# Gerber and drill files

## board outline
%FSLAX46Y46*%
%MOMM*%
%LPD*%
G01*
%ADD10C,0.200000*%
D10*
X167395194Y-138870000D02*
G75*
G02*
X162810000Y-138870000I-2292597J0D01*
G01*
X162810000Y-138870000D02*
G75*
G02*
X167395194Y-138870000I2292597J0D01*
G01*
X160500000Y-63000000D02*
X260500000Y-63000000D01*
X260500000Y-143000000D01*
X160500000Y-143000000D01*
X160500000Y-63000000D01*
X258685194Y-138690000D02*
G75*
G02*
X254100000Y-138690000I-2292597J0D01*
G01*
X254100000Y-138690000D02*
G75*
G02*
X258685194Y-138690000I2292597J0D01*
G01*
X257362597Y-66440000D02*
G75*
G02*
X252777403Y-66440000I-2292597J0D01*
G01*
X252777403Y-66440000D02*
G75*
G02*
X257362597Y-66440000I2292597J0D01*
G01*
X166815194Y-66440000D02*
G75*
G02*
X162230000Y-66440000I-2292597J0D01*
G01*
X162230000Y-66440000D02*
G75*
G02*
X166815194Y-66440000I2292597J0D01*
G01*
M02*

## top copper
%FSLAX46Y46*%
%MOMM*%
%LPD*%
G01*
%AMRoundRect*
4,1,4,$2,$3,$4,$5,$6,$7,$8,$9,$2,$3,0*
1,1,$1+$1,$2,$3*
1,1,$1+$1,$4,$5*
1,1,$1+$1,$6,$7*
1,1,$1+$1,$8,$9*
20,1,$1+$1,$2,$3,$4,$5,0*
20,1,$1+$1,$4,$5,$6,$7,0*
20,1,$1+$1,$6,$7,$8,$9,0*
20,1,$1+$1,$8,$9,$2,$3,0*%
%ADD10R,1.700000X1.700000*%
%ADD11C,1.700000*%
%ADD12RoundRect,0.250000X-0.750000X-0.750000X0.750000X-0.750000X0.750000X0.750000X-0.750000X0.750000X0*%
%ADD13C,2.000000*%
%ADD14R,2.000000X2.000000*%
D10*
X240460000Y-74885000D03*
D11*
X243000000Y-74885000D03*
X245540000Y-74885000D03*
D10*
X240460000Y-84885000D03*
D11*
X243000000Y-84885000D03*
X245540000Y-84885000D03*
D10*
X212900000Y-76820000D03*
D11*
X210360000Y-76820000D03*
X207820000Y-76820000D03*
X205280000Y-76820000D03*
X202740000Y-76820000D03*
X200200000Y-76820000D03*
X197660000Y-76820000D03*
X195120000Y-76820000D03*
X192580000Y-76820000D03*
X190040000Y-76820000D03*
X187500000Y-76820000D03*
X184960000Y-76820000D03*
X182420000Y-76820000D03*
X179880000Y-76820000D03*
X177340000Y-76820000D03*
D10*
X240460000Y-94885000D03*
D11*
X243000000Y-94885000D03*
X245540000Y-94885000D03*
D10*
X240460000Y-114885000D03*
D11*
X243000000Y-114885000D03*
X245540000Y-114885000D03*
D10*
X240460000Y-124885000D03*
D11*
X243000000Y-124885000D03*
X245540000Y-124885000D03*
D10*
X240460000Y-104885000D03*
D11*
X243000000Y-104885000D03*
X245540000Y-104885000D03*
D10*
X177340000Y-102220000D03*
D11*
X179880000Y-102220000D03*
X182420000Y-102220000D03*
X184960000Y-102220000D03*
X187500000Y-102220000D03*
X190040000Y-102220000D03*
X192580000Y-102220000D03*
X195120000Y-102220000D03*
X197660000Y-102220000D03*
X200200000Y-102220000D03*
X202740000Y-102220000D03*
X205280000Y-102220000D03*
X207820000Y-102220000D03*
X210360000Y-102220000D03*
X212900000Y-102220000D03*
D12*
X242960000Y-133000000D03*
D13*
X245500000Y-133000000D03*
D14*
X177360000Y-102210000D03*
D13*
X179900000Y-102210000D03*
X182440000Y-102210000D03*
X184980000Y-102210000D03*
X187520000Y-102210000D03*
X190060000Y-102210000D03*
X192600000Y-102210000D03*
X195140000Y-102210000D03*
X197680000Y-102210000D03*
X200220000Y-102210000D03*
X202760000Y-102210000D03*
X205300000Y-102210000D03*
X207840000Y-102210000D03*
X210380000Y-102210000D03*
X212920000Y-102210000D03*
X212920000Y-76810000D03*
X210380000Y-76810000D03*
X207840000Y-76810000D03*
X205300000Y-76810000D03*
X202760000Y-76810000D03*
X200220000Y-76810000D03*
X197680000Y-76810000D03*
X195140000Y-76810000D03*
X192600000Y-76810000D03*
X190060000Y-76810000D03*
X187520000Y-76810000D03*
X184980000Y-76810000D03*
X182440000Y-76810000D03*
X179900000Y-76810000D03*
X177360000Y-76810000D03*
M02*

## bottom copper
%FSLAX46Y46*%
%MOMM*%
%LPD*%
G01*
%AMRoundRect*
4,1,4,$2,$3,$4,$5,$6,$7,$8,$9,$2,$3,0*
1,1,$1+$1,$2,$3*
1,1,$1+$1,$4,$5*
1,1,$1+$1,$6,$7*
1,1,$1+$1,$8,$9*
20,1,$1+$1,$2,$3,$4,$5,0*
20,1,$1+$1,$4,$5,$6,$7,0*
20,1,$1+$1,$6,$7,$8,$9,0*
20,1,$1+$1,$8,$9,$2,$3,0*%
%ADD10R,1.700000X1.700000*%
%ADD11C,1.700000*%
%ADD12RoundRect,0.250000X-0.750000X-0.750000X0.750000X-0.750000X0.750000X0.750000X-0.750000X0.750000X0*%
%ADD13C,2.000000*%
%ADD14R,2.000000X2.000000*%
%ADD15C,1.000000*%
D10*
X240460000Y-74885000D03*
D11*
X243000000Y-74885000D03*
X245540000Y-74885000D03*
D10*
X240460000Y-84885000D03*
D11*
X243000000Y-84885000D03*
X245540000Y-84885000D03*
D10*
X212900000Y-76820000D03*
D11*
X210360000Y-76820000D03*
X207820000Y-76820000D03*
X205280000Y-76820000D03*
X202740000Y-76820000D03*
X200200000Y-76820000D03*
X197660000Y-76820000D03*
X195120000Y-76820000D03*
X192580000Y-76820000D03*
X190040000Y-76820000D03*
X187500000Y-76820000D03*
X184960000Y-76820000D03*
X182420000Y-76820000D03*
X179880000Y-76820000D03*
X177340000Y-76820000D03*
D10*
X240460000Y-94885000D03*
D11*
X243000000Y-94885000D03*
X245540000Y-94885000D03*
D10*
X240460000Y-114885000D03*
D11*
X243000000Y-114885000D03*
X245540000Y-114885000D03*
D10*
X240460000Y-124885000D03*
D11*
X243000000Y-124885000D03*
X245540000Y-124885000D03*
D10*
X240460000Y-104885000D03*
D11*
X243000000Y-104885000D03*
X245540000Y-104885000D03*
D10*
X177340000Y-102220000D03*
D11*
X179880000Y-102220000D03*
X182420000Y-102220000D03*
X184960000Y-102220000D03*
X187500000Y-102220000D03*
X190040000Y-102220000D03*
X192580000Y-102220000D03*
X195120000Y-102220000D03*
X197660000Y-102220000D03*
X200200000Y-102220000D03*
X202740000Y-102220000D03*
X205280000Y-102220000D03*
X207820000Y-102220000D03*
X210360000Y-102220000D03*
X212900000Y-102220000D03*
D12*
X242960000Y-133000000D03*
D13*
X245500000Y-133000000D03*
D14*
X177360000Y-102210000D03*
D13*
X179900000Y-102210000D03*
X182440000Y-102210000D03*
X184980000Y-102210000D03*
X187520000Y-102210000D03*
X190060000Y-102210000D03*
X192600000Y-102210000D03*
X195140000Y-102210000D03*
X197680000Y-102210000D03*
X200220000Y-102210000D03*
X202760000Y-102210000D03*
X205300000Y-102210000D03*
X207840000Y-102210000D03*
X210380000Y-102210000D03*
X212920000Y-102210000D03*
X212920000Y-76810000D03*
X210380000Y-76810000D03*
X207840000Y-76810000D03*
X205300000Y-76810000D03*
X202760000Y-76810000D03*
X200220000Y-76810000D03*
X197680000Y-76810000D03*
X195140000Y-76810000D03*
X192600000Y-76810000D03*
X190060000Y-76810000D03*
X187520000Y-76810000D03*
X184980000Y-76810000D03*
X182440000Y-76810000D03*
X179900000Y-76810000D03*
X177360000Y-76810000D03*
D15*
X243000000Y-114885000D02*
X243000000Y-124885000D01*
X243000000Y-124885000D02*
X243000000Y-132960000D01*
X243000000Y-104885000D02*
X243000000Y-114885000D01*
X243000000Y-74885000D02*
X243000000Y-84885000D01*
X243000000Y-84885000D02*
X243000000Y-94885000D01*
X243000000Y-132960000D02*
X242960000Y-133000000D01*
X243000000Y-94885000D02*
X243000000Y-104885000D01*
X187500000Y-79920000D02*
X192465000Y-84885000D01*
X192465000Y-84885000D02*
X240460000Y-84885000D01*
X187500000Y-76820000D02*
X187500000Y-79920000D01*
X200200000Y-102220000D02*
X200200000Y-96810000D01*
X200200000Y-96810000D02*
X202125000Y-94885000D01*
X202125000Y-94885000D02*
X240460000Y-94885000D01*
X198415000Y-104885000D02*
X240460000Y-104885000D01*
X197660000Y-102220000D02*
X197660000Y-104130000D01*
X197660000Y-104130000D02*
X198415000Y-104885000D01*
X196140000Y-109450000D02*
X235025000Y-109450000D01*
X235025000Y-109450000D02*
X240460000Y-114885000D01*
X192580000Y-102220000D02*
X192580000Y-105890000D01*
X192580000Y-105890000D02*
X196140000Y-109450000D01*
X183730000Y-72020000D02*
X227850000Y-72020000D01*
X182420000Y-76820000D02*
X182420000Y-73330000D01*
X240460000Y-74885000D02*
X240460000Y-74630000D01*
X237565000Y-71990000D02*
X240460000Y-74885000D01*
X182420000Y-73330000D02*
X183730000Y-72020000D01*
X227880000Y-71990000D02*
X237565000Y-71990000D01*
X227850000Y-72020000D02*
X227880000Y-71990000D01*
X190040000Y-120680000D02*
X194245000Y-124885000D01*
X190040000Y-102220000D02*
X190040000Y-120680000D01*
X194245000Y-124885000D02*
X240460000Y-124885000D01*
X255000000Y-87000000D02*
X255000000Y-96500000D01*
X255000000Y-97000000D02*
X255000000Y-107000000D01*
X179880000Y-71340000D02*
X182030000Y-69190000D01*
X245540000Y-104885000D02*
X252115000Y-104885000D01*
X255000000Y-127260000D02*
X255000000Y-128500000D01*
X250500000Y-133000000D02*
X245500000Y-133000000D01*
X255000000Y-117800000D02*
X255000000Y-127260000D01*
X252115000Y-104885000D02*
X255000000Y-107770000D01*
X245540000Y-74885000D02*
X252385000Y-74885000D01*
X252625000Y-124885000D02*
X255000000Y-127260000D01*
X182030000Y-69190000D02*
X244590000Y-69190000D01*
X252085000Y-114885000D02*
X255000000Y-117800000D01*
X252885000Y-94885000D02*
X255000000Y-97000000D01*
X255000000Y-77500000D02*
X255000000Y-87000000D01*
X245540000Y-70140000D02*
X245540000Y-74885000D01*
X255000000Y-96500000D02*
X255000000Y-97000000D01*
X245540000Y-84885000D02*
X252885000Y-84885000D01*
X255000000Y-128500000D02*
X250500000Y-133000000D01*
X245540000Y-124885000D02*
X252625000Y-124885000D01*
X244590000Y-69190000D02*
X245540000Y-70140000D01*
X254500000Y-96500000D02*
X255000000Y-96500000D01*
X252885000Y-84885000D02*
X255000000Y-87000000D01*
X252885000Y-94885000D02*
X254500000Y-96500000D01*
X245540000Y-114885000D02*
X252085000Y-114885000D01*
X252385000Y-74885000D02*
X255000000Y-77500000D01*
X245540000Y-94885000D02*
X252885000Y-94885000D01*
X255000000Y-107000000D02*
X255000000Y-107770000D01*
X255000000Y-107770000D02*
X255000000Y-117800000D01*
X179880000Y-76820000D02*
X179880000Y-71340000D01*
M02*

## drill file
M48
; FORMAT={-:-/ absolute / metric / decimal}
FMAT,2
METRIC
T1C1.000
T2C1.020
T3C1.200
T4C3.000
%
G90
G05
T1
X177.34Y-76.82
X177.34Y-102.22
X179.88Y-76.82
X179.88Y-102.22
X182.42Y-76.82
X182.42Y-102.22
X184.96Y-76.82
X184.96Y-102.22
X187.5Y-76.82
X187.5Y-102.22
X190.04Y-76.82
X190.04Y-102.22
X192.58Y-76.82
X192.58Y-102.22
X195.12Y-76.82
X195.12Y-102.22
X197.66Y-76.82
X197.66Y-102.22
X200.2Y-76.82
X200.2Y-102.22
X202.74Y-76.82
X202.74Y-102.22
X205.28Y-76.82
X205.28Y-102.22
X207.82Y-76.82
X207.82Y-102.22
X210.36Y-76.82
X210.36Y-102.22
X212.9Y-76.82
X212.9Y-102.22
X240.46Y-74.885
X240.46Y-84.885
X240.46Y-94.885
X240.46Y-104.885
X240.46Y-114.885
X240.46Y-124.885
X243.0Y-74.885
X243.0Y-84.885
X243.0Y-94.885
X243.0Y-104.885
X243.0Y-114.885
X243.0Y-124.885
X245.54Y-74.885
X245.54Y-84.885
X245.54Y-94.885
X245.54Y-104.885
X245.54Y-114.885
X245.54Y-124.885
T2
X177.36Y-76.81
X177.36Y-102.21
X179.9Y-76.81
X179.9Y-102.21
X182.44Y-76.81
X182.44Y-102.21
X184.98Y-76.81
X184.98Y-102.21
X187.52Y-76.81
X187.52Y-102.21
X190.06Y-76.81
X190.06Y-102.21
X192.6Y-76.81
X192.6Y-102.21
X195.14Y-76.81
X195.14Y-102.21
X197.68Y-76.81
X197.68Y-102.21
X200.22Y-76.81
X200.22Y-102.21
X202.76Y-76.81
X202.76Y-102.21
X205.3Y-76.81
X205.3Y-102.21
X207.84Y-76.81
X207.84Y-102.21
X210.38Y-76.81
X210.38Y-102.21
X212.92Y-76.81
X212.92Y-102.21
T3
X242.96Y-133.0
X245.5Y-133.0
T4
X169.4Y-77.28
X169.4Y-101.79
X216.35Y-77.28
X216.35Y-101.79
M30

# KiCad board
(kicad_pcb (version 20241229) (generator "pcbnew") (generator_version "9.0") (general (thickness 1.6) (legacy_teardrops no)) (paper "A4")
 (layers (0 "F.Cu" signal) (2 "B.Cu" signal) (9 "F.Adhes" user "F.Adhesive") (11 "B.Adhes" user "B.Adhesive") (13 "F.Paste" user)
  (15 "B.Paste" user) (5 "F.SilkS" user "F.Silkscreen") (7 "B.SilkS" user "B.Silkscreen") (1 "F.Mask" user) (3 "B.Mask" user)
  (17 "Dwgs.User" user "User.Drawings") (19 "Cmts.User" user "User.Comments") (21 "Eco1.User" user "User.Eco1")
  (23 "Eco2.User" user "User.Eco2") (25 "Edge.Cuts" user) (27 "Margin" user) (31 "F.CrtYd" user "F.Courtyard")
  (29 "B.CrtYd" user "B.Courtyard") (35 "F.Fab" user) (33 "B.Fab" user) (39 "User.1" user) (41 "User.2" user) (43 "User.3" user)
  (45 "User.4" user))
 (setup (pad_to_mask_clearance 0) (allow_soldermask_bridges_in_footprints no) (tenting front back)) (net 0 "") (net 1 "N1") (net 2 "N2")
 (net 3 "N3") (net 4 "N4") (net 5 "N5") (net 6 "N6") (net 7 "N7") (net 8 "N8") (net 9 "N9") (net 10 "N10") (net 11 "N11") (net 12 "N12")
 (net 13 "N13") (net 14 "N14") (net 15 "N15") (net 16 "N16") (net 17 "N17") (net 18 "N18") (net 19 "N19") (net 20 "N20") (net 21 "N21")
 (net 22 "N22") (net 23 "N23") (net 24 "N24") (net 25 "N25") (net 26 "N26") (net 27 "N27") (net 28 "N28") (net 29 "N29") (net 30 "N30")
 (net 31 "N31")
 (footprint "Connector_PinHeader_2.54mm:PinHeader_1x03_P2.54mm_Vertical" (layer "F.Cu") (at 240.46 74.885 90)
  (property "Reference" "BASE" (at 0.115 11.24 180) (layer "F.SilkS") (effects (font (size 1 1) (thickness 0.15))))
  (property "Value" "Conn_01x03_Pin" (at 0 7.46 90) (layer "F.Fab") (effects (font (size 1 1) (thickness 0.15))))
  (pad "1" thru_hole rect (at 0 0 90) (size 1.7 1.7) (drill 1) (layers "*.Cu" "*.Mask") (remove_unused_layers no) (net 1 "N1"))
  (pad "2" thru_hole circle (at 0 2.54 90) (size 1.7 1.7) (drill 1) (layers "*.Cu" "*.Mask") (remove_unused_layers no) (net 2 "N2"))
  (pad "3" thru_hole circle (at 0 5.08 90) (size 1.7 1.7) (drill 1) (layers "*.Cu" "*.Mask") (remove_unused_layers no) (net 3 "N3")))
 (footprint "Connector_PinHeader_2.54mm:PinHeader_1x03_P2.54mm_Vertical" (layer "F.Cu") (at 240.46 84.885 90)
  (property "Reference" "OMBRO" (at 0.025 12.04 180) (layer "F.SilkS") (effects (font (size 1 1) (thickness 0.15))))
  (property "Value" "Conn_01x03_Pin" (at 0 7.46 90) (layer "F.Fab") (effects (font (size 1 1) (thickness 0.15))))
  (pad "1" thru_hole rect (at 0 0 90) (size 1.7 1.7) (drill 1) (layers "*.Cu" "*.Mask") (remove_unused_layers no) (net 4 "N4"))
  (pad "2" thru_hole circle (at 0 2.54 90) (size 1.7 1.7) (drill 1) (layers "*.Cu" "*.Mask") (remove_unused_layers no) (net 2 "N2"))
  (pad "3" thru_hole circle (at 0 5.08 90) (size 1.7 1.7) (drill 1) (layers "*.Cu" "*.Mask") (remove_unused_layers no) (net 3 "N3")))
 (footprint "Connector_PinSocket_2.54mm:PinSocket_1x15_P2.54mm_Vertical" (layer "F.Cu") (at 212.9 76.82 -90)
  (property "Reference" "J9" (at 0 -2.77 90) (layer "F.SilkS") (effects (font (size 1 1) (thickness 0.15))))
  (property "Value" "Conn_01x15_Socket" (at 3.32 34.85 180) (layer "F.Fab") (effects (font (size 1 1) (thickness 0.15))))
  (pad "1" thru_hole rect (at 0 0 270) (size 1.7 1.7) (drill 1) (layers "*.Cu" "*.Mask") (remove_unused_layers no) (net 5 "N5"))
  (pad "2" thru_hole circle (at 0 2.54 270) (size 1.7 1.7) (drill 1) (layers "*.Cu" "*.Mask") (remove_unused_layers no) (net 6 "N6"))
  (pad "3" thru_hole circle (at 0 5.08 270) (size 1.7 1.7) (drill 1) (layers "*.Cu" "*.Mask") (remove_unused_layers no) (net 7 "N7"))
  (pad "4" thru_hole circle (at 0 7.62 270) (size 1.7 1.7) (drill 1) (layers "*.Cu" "*.Mask") (remove_unused_layers no) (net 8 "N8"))
  (pad "5" thru_hole circle (at 0 10.16 270) (size 1.7 1.7) (drill 1) (layers "*.Cu" "*.Mask") (remove_unused_layers no) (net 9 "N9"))
  (pad "6" thru_hole circle (at 0 12.7 270) (size 1.7 1.7) (drill 1) (layers "*.Cu" "*.Mask") (remove_unused_layers no) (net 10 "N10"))
  (pad "7" thru_hole circle (at 0 15.24 270) (size 1.7 1.7) (drill 1) (layers "*.Cu" "*.Mask") (remove_unused_layers no) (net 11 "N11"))
  (pad "8" thru_hole circle (at 0 17.78 270) (size 1.7 1.7) (drill 1) (layers "*.Cu" "*.Mask") (remove_unused_layers no) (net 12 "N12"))
  (pad "9" thru_hole circle (at 0 20.32 270) (size 1.7 1.7) (drill 1) (layers "*.Cu" "*.Mask") (remove_unused_layers no) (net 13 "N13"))
  (pad "10" thru_hole circle (at 0 22.86 270) (size 1.7 1.7) (drill 1) (layers "*.Cu" "*.Mask") (remove_unused_layers no) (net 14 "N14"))
  (pad "11" thru_hole circle (at 0 25.4 270) (size 1.7 1.7) (drill 1) (layers "*.Cu" "*.Mask") (remove_unused_layers no) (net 4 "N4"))
  (pad "12" thru_hole circle (at 0 27.94 270) (size 1.7 1.7) (drill 1) (layers "*.Cu" "*.Mask") (remove_unused_layers no) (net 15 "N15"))
  (pad "13" thru_hole circle (at 0 30.48 270) (size 1.7 1.7) (drill 1) (layers "*.Cu" "*.Mask") (remove_unused_layers no) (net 1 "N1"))
  (pad "14" thru_hole circle (at 0 33.02 270) (size 1.7 1.7) (drill 1) (layers "*.Cu" "*.Mask") (remove_unused_layers no) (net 3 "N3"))
  (pad "15" thru_hole circle (at 0 35.56 270) (size 1.7 1.7) (drill 1) (layers "*.Cu" "*.Mask") (remove_unused_layers no) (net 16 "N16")))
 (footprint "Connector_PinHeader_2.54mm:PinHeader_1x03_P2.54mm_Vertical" (layer "F.Cu") (at 240.46 94.885 90)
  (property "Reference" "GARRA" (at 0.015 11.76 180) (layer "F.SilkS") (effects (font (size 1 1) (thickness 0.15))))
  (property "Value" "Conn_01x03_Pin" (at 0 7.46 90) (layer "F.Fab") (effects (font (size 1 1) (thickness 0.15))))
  (pad "1" thru_hole rect (at 0 0 90) (size 1.7 1.7) (drill 1) (layers "*.Cu" "*.Mask") (remove_unused_layers no) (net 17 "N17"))
  (pad "2" thru_hole circle (at 0 2.54 90) (size 1.7 1.7) (drill 1) (layers "*.Cu" "*.Mask") (remove_unused_layers no) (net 2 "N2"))
  (pad "3" thru_hole circle (at 0 5.08 90) (size 1.7 1.7) (drill 1) (layers "*.Cu" "*.Mask") (remove_unused_layers no) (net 3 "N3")))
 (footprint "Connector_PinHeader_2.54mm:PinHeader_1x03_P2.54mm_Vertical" (layer "F.Cu") (at 240.46 114.885 90)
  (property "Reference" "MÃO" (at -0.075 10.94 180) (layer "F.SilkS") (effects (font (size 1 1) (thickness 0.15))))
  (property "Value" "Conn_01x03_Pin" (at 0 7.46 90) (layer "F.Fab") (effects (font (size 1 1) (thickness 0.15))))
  (pad "1" thru_hole rect (at 0 0 90) (size 1.7 1.7) (drill 1) (layers "*.Cu" "*.Mask") (remove_unused_layers no) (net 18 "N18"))
  (pad "2" thru_hole circle (at 0 2.54 90) (size 1.7 1.7) (drill 1) (layers "*.Cu" "*.Mask") (remove_unused_layers no) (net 2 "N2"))
  (pad "3" thru_hole circle (at 0 5.08 90) (size 1.7 1.7) (drill 1) (layers "*.Cu" "*.Mask") (remove_unused_layers no) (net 3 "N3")))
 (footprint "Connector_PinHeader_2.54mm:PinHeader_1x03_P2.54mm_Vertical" (layer "F.Cu") (at 240.46 124.885 90)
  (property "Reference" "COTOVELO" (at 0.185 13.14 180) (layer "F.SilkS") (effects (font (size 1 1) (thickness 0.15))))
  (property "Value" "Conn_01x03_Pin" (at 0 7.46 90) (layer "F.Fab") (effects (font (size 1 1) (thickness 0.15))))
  (pad "1" thru_hole rect (at 0 0 90) (size 1.7 1.7) (drill 1) (layers "*.Cu" "*.Mask") (remove_unused_layers no) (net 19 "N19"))
  (pad "2" thru_hole circle (at 0 2.54 90) (size 1.7 1.7) (drill 1) (layers "*.Cu" "*.Mask") (remove_unused_layers no) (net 2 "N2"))
  (pad "3" thru_hole circle (at 0 5.08 90) (size 1.7 1.7) (drill 1) (layers "*.Cu" "*.Mask") (remove_unused_layers no) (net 3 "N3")))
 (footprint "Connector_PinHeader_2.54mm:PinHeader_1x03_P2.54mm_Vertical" (layer "F.Cu") (at 240.46 104.885 90)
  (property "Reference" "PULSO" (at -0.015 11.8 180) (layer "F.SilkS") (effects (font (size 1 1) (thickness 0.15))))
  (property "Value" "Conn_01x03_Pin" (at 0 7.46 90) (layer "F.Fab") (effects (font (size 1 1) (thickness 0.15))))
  (pad "1" thru_hole rect (at 0 0 90) (size 1.7 1.7) (drill 1) (layers "*.Cu" "*.Mask") (remove_unused_layers no) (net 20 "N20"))
  (pad "2" thru_hole circle (at 0 2.54 90) (size 1.7 1.7) (drill 1) (layers "*.Cu" "*.Mask") (remove_unused_layers no) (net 2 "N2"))
  (pad "3" thru_hole circle (at 0 5.08 90) (size 1.7 1.7) (drill 1) (layers "*.Cu" "*.Mask") (remove_unused_layers no) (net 3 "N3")))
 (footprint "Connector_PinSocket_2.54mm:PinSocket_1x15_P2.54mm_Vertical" (layer "F.Cu") (at 177.34 102.22 90)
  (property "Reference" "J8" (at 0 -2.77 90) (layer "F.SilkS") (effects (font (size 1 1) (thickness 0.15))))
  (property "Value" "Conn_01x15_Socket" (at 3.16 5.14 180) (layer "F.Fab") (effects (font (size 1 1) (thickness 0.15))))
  (pad "1" thru_hole rect (at 0 0 90) (size 1.7 1.7) (drill 1) (layers "*.Cu" "*.Mask") (remove_unused_layers no) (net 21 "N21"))
  (pad "2" thru_hole circle (at 0 2.54 90) (size 1.7 1.7) (drill 1) (layers "*.Cu" "*.Mask") (remove_unused_layers no) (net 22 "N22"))
  (pad "3" thru_hole circle (at 0 5.08 90) (size 1.7 1.7) (drill 1) (layers "*.Cu" "*.Mask") (remove_unused_layers no) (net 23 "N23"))
  (pad "4" thru_hole circle (at 0 7.62 90) (size 1.7 1.7) (drill 1) (layers "*.Cu" "*.Mask") (remove_unused_layers no) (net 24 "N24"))
  (pad "5" thru_hole circle (at 0 10.16 90) (size 1.7 1.7) (drill 1) (layers "*.Cu" "*.Mask") (remove_unused_layers no) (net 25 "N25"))
  (pad "6" thru_hole circle (at 0 12.7 90) (size 1.7 1.7) (drill 1) (layers "*.Cu" "*.Mask") (remove_unused_layers no) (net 19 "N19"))
  (pad "7" thru_hole circle (at 0 15.24 90) (size 1.7 1.7) (drill 1) (layers "*.Cu" "*.Mask") (remove_unused_layers no) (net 18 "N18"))
  (pad "8" thru_hole circle (at 0 17.78 90) (size 1.7 1.7) (drill 1) (layers "*.Cu" "*.Mask") (remove_unused_layers no) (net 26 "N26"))
  (pad "9" thru_hole circle (at 0 20.32 90) (size 1.7 1.7) (drill 1) (layers "*.Cu" "*.Mask") (remove_unused_layers no) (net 20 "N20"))
  (pad "10" thru_hole circle (at 0 22.86 90) (size 1.7 1.7) (drill 1) (layers "*.Cu" "*.Mask") (remove_unused_layers no) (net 17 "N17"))
  (pad "11" thru_hole circle (at 0 25.4 90) (size 1.7 1.7) (drill 1) (layers "*.Cu" "*.Mask") (remove_unused_layers no) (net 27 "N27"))
  (pad "12" thru_hole circle (at 0 27.94 90) (size 1.7 1.7) (drill 1) (layers "*.Cu" "*.Mask") (remove_unused_layers no) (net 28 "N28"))
  (pad "13" thru_hole circle (at 0 30.48 90) (size 1.7 1.7) (drill 1) (layers "*.Cu" "*.Mask") (remove_unused_layers no) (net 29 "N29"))
  (pad "14" thru_hole circle (at 0 33.02 90) (size 1.7 1.7) (drill 1) (layers "*.Cu" "*.Mask") (remove_unused_layers no) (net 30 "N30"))
  (pad "15" thru_hole circle (at 0 35.56 90) (size 1.7 1.7) (drill 1) (layers "*.Cu" "*.Mask") (remove_unused_layers no) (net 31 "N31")))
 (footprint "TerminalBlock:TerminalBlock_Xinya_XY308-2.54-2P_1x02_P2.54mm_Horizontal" (layer "F.Cu") (at 242.96 133)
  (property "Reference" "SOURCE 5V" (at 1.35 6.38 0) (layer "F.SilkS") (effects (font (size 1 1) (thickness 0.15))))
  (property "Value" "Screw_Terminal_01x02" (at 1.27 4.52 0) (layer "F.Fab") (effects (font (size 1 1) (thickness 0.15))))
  (pad "1" thru_hole roundrect (at 0 0) (size 2 2) (drill 1.2) (layers "*.Cu" "*.Mask") (remove_unused_layers no) (roundrect_rratio 0.125)
   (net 2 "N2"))
  (pad "2" thru_hole circle (at 2.54 0) (size 2 2) (drill 1.2) (layers "*.Cu" "*.Mask") (remove_unused_layers no) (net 3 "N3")))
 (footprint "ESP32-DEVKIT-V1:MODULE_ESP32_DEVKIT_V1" (layer "F.Cu") (at 192.875 89.51 90)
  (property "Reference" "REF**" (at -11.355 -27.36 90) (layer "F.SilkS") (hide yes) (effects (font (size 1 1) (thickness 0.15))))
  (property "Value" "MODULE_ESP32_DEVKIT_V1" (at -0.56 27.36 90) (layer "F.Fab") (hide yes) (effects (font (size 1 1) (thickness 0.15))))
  (pad "" np_thru_hole circle (at -12.28 -23.475 90) (size 3 3) (drill 3) (layers "*.Cu" "*.Mask"))
  (pad "" np_thru_hole circle (at -12.28 23.475 90) (size 3 3) (drill 3) (layers "*.Cu" "*.Mask"))
  (pad "" np_thru_hole circle (at 12.23 -23.475 90) (size 3 3) (drill 3) (layers "*.Cu" "*.Mask"))
  (pad "" np_thru_hole circle (at 12.23 23.475 90) (size 3 3) (drill 3) (layers "*.Cu" "*.Mask"))
  (pad "1" thru_hole rect (at -12.7 -15.515 90) (size 2 2) (drill 1.02) (layers "*.Cu" "*.Mask") (remove_unused_layers no)
   (solder_mask_margin 0.102))
  (pad "2" thru_hole circle (at -12.7 -12.975 90) (size 2 2) (drill 1.02) (layers "*.Cu" "*.Mask") (remove_unused_layers no)
   (solder_mask_margin 0.102))
  (pad "3" thru_hole circle (at -12.7 -10.435 90) (size 2 2) (drill 1.02) (layers "*.Cu" "*.Mask") (remove_unused_layers no)
   (solder_mask_margin 0.102))
  (pad "4" thru_hole circle (at -12.7 -7.895 90) (size 2 2) (drill 1.02) (layers "*.Cu" "*.Mask") (remove_unused_layers no)
   (solder_mask_margin 0.102))
  (pad "5" thru_hole circle (at -12.7 -5.355 90) (size 2 2) (drill 1.02) (layers "*.Cu" "*.Mask") (remove_unused_layers no)
   (solder_mask_margin 0.102))
  (pad "6" thru_hole circle (at -12.7 -2.815 90) (size 2 2) (drill 1.02) (layers "*.Cu" "*.Mask") (remove_unused_layers no)
   (solder_mask_margin 0.102))
  (pad "7" thru_hole circle (at -12.7 -0.275 90) (size 2 2) (drill 1.02) (layers "*.Cu" "*.Mask") (remove_unused_layers no)
   (solder_mask_margin 0.102))
  (pad "8" thru_hole circle (at -12.7 2.265 90) (size 2 2) (drill 1.02) (layers "*.Cu" "*.Mask") (remove_unused_layers no)
   (solder_mask_margin 0.102))
  (pad "9" thru_hole circle (at -12.7 4.805 90) (size 2 2) (drill 1.02) (layers "*.Cu" "*.Mask") (remove_unused_layers no)
   (solder_mask_margin 0.102))
  (pad "10" thru_hole circle (at -12.7 7.345 90) (size 2 2) (drill 1.02) (layers "*.Cu" "*.Mask") (remove_unused_layers no)
   (solder_mask_margin 0.102))
  (pad "11" thru_hole circle (at -12.7 9.885 90) (size 2 2) (drill 1.02) (layers "*.Cu" "*.Mask") (remove_unused_layers no)
   (solder_mask_margin 0.102))
  (pad "12" thru_hole circle (at -12.7 12.425 90) (size 2 2) (drill 1.02) (layers "*.Cu" "*.Mask") (remove_unused_layers no)
   (solder_mask_margin 0.102))
  (pad "13" thru_hole circle (at -12.7 14.965 90) (size 2 2) (drill 1.02) (layers "*.Cu" "*.Mask") (remove_unused_layers no)
   (solder_mask_margin 0.102))
  (pad "14" thru_hole circle (at -12.7 17.505 90) (size 2 2) (drill 1.02) (layers "*.Cu" "*.Mask") (remove_unused_layers no)
   (solder_mask_margin 0.102))
  (pad "15" thru_hole circle (at -12.7 20.045 90) (size 2 2) (drill 1.02) (layers "*.Cu" "*.Mask") (remove_unused_layers no)
   (solder_mask_margin 0.102))
  (pad "16" thru_hole circle (at 12.7 20.045 90) (size 2 2) (drill 1.02) (layers "*.Cu" "*.Mask") (remove_unused_layers no)
   (solder_mask_margin 0.102))
  (pad "17" thru_hole circle (at 12.7 17.505 90) (size 2 2) (drill 1.02) (layers "*.Cu" "*.Mask") (remove_unused_layers no)
   (solder_mask_margin 0.102))
  (pad "18" thru_hole circle (at 12.7 14.965 90) (size 2 2) (drill 1.02) (layers "*.Cu" "*.Mask") (remove_unused_layers no)
   (solder_mask_margin 0.102))
  (pad "19" thru_hole circle (at 12.7 12.425 90) (size 2 2) (drill 1.02) (layers "*.Cu" "*.Mask") (remove_unused_layers no)
   (solder_mask_margin 0.102))
  (pad "20" thru_hole circle (at 12.7 9.885 90) (size 2 2) (drill 1.02) (layers "*.Cu" "*.Mask") (remove_unused_layers no)
   (solder_mask_margin 0.102))
  (pad "21" thru_hole circle (at 12.7 7.345 90) (size 2 2) (drill 1.02) (layers "*.Cu" "*.Mask") (remove_unused_layers no)
   (solder_mask_margin 0.102))
  (pad "22" thru_hole circle (at 12.7 4.805 90) (size 2 2) (drill 1.02) (layers "*.Cu" "*.Mask") (remove_unused_layers no)
   (solder_mask_margin 0.102))
  (pad "23" thru_hole circle (at 12.7 2.265 90) (size 2 2) (drill 1.02) (layers "*.Cu" "*.Mask") (remove_unused_layers no)
   (solder_mask_margin 0.102))
  (pad "24" thru_hole circle (at 12.7 -0.275 90) (size 2 2) (drill 1.02) (layers "*.Cu" "*.Mask") (remove_unused_layers no)
   (solder_mask_margin 0.102))
  (pad "25" thru_hole circle (at 12.7 -2.815 90) (size 2 2) (drill 1.02) (layers "*.Cu" "*.Mask") (remove_unused_layers no)
   (solder_mask_margin 0.102))
  (pad "26" thru_hole circle (at 12.7 -5.355 90) (size 2 2) (drill 1.02) (layers "*.Cu" "*.Mask") (remove_unused_layers no)
   (solder_mask_margin 0.102))
  (pad "27" thru_hole circle (at 12.7 -7.895 90) (size 2 2) (drill 1.02) (layers "*.Cu" "*.Mask") (remove_unused_layers no)
   (solder_mask_margin 0.102))
  (pad "28" thru_hole circle (at 12.7 -10.435 90) (size 2 2) (drill 1.02) (layers "*.Cu" "*.Mask") (remove_unused_layers no)
   (solder_mask_margin 0.102))
  (pad "29" thru_hole circle (at 12.7 -12.975 90) (size 2 2) (drill 1.02) (layers "*.Cu" "*.Mask") (remove_unused_layers no)
   (solder_mask_margin 0.102))
  (pad "30" thru_hole circle (at 12.7 -15.515 90) (size 2 2) (drill 1.02) (layers "*.Cu" "*.Mask") (remove_unused_layers no)
   (solder_mask_margin 0.102))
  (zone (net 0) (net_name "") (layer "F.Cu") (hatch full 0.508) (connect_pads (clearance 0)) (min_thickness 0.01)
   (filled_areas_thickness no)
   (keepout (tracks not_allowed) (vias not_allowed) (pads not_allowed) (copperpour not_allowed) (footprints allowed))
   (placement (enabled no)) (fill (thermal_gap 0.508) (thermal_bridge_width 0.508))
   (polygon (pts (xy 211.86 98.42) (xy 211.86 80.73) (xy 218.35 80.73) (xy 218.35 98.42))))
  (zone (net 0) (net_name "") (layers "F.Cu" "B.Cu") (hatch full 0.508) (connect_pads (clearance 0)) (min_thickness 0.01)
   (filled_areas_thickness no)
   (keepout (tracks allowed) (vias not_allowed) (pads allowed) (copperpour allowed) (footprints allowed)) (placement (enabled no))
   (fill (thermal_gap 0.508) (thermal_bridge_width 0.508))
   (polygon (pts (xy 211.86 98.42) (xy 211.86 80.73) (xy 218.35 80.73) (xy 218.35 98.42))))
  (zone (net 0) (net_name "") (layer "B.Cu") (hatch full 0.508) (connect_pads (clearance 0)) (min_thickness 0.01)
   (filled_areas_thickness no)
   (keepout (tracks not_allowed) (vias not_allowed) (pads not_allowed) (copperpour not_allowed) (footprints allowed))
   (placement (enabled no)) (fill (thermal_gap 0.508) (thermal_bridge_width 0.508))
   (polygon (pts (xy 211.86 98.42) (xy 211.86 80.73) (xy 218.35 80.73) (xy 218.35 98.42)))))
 (gr_circle (center 165.102597 138.87) (end 166.782597 140.43) (stroke (width 0.2) (type solid)) (fill no) (layer "Edge.Cuts"))
 (gr_rect (start 160.5 63) (end 260.5 143) (stroke (width 0.2) (type solid)) (fill no) (layer "Edge.Cuts"))
 (gr_circle (center 256.392597 138.69) (end 258.072597 140.25) (stroke (width 0.2) (type solid)) (fill no) (layer "Edge.Cuts"))
 (gr_circle (center 255.07 66.44) (end 256.75 68) (stroke (width 0.2) (type solid)) (fill no) (layer "Edge.Cuts"))
 (gr_circle (center 164.522597 66.44) (end 166.202597 68) (stroke (width 0.2) (type solid)) (fill no) (layer "Edge.Cuts"))
 (segment (start 243 114.885) (end 243 124.885) (width 1) (layer "B.Cu") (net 2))
 (segment (start 243 124.885) (end 243 132.96) (width 1) (layer "B.Cu") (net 2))
 (segment (start 243 104.885) (end 243 114.885) (width 1) (layer "B.Cu") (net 2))
 (segment (start 243 74.885) (end 243 84.885) (width 1) (layer "B.Cu") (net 2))
 (segment (start 243 84.885) (end 243 94.885) (width 1) (layer "B.Cu") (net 2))
 (segment (start 243 132.96) (end 242.96 133) (width 1) (layer "B.Cu") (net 2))
 (segment (start 243 94.885) (end 243 104.885) (width 1) (layer "B.Cu") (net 2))
 (segment (start 187.5 79.92) (end 192.465 84.885) (width 1) (layer "B.Cu") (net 4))
 (segment (start 192.465 84.885) (end 240.46 84.885) (width 1) (layer "B.Cu") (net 4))
 (segment (start 187.5 76.82) (end 187.5 79.92) (width 1) (layer "B.Cu") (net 4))
 (segment (start 200.2 102.22) (end 200.2 96.81) (width 1) (layer "B.Cu") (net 17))
 (segment (start 200.2 96.81) (end 202.125 94.885) (width 1) (layer "B.Cu") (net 17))
 (segment (start 202.125 94.885) (end 240.46 94.885) (width 1) (layer "B.Cu") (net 17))
 (segment (start 198.415 104.885) (end 240.46 104.885) (width 1) (layer "B.Cu") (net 20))
 (segment (start 197.66 102.22) (end 197.66 104.13) (width 1) (layer "B.Cu") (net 20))
 (segment (start 197.66 104.13) (end 198.415 104.885) (width 1) (layer "B.Cu") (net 20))
 (segment (start 196.14 109.45) (end 235.025 109.45) (width 1) (layer "B.Cu") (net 18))
 (segment (start 235.025 109.45) (end 240.46 114.885) (width 1) (layer "B.Cu") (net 18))
 (segment (start 192.58 102.22) (end 192.58 105.89) (width 1) (layer "B.Cu") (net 18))
 (segment (start 192.58 105.89) (end 196.14 109.45) (width 1) (layer "B.Cu") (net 18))
 (segment (start 183.73 72.02) (end 227.85 72.02) (width 1) (layer "B.Cu") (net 1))
 (segment (start 182.42 76.82) (end 182.42 73.33) (width 1) (layer "B.Cu") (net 1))
 (segment (start 240.46 74.885) (end 240.46 74.63) (width 1) (layer "B.Cu") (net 1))
 (segment (start 237.565 71.99) (end 240.46 74.885) (width 1) (layer "B.Cu") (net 1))
 (segment (start 182.42 73.33) (end 183.73 72.02) (width 1) (layer "B.Cu") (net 1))
 (segment (start 227.88 71.99) (end 237.565 71.99) (width 1) (layer "B.Cu") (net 1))
 (segment (start 227.85 72.02) (end 227.88 71.99) (width 1) (layer "B.Cu") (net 1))
 (segment (start 190.04 120.68) (end 194.245 124.885) (width 1) (layer "B.Cu") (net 19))
 (segment (start 190.04 102.22) (end 190.04 120.68) (width 1) (layer "B.Cu") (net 19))
 (segment (start 194.245 124.885) (end 240.46 124.885) (width 1) (layer "B.Cu") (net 19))
 (segment (start 255 87) (end 255 96.5) (width 1) (layer "B.Cu") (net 3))
 (segment (start 255 97) (end 255 107) (width 1) (layer "B.Cu") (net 3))
 (segment (start 179.88 71.34) (end 182.03 69.19) (width 1) (layer "B.Cu") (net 3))
 (segment (start 245.54 104.885) (end 252.115 104.885) (width 1) (layer "B.Cu") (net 3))
 (segment (start 255 127.26) (end 255 128.5) (width 1) (layer "B.Cu") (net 3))
 (segment (start 250.5 133) (end 245.5 133) (width 1) (layer "B.Cu") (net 3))
 (segment (start 255 117.8) (end 255 127.26) (width 1) (layer "B.Cu") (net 3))
 (segment (start 252.115 104.885) (end 255 107.77) (width 1) (layer "B.Cu") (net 3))
 (segment (start 245.54 74.885) (end 252.385 74.885) (width 1) (layer "B.Cu") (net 3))
 (segment (start 252.625 124.885) (end 255 127.26) (width 1) (layer "B.Cu") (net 3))
 (segment (start 182.03 69.19) (end 244.59 69.19) (width 1) (layer "B.Cu") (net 3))
 (segment (start 252.085 114.885) (end 255 117.8) (width 1) (layer "B.Cu") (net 3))
 (segment (start 252.885 94.885) (end 255 97) (width 1) (layer "B.Cu") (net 3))
 (segment (start 255 77.5) (end 255 87) (width 1) (layer "B.Cu") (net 3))
 (segment (start 245.54 70.14) (end 245.54 74.885) (width 1) (layer "B.Cu") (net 3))
 (segment (start 255 96.5) (end 255 97) (width 1) (layer "B.Cu") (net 3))
 (segment (start 245.54 84.885) (end 252.885 84.885) (width 1) (layer "B.Cu") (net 3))
 (segment (start 255 128.5) (end 250.5 133) (width 1) (layer "B.Cu") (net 3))
 (segment (start 245.54 124.885) (end 252.625 124.885) (width 1) (layer "B.Cu") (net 3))
 (segment (start 244.59 69.19) (end 245.54 70.14) (width 1) (layer "B.Cu") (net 3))
 (segment (start 254.5 96.5) (end 255 96.5) (width 1) (layer "B.Cu") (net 3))
 (segment (start 252.885 84.885) (end 255 87) (width 1) (layer "B.Cu") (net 3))
 (segment (start 252.885 94.885) (end 254.5 96.5) (width 1) (layer "B.Cu") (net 3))
 (segment (start 245.54 114.885) (end 252.085 114.885) (width 1) (layer "B.Cu") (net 3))
 (segment (start 252.385 74.885) (end 255 77.5) (width 1) (layer "B.Cu") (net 3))
 (segment (start 245.54 94.885) (end 252.885 94.885) (width 1) (layer "B.Cu") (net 3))
 (segment (start 255 107) (end 255 107.77) (width 1) (layer "B.Cu") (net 3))
 (segment (start 255 107.77) (end 255 117.8) (width 1) (layer "B.Cu") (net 3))
 (segment (start 179.88 76.82) (end 179.88 71.34) (width 1) (layer "B.Cu") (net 3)))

